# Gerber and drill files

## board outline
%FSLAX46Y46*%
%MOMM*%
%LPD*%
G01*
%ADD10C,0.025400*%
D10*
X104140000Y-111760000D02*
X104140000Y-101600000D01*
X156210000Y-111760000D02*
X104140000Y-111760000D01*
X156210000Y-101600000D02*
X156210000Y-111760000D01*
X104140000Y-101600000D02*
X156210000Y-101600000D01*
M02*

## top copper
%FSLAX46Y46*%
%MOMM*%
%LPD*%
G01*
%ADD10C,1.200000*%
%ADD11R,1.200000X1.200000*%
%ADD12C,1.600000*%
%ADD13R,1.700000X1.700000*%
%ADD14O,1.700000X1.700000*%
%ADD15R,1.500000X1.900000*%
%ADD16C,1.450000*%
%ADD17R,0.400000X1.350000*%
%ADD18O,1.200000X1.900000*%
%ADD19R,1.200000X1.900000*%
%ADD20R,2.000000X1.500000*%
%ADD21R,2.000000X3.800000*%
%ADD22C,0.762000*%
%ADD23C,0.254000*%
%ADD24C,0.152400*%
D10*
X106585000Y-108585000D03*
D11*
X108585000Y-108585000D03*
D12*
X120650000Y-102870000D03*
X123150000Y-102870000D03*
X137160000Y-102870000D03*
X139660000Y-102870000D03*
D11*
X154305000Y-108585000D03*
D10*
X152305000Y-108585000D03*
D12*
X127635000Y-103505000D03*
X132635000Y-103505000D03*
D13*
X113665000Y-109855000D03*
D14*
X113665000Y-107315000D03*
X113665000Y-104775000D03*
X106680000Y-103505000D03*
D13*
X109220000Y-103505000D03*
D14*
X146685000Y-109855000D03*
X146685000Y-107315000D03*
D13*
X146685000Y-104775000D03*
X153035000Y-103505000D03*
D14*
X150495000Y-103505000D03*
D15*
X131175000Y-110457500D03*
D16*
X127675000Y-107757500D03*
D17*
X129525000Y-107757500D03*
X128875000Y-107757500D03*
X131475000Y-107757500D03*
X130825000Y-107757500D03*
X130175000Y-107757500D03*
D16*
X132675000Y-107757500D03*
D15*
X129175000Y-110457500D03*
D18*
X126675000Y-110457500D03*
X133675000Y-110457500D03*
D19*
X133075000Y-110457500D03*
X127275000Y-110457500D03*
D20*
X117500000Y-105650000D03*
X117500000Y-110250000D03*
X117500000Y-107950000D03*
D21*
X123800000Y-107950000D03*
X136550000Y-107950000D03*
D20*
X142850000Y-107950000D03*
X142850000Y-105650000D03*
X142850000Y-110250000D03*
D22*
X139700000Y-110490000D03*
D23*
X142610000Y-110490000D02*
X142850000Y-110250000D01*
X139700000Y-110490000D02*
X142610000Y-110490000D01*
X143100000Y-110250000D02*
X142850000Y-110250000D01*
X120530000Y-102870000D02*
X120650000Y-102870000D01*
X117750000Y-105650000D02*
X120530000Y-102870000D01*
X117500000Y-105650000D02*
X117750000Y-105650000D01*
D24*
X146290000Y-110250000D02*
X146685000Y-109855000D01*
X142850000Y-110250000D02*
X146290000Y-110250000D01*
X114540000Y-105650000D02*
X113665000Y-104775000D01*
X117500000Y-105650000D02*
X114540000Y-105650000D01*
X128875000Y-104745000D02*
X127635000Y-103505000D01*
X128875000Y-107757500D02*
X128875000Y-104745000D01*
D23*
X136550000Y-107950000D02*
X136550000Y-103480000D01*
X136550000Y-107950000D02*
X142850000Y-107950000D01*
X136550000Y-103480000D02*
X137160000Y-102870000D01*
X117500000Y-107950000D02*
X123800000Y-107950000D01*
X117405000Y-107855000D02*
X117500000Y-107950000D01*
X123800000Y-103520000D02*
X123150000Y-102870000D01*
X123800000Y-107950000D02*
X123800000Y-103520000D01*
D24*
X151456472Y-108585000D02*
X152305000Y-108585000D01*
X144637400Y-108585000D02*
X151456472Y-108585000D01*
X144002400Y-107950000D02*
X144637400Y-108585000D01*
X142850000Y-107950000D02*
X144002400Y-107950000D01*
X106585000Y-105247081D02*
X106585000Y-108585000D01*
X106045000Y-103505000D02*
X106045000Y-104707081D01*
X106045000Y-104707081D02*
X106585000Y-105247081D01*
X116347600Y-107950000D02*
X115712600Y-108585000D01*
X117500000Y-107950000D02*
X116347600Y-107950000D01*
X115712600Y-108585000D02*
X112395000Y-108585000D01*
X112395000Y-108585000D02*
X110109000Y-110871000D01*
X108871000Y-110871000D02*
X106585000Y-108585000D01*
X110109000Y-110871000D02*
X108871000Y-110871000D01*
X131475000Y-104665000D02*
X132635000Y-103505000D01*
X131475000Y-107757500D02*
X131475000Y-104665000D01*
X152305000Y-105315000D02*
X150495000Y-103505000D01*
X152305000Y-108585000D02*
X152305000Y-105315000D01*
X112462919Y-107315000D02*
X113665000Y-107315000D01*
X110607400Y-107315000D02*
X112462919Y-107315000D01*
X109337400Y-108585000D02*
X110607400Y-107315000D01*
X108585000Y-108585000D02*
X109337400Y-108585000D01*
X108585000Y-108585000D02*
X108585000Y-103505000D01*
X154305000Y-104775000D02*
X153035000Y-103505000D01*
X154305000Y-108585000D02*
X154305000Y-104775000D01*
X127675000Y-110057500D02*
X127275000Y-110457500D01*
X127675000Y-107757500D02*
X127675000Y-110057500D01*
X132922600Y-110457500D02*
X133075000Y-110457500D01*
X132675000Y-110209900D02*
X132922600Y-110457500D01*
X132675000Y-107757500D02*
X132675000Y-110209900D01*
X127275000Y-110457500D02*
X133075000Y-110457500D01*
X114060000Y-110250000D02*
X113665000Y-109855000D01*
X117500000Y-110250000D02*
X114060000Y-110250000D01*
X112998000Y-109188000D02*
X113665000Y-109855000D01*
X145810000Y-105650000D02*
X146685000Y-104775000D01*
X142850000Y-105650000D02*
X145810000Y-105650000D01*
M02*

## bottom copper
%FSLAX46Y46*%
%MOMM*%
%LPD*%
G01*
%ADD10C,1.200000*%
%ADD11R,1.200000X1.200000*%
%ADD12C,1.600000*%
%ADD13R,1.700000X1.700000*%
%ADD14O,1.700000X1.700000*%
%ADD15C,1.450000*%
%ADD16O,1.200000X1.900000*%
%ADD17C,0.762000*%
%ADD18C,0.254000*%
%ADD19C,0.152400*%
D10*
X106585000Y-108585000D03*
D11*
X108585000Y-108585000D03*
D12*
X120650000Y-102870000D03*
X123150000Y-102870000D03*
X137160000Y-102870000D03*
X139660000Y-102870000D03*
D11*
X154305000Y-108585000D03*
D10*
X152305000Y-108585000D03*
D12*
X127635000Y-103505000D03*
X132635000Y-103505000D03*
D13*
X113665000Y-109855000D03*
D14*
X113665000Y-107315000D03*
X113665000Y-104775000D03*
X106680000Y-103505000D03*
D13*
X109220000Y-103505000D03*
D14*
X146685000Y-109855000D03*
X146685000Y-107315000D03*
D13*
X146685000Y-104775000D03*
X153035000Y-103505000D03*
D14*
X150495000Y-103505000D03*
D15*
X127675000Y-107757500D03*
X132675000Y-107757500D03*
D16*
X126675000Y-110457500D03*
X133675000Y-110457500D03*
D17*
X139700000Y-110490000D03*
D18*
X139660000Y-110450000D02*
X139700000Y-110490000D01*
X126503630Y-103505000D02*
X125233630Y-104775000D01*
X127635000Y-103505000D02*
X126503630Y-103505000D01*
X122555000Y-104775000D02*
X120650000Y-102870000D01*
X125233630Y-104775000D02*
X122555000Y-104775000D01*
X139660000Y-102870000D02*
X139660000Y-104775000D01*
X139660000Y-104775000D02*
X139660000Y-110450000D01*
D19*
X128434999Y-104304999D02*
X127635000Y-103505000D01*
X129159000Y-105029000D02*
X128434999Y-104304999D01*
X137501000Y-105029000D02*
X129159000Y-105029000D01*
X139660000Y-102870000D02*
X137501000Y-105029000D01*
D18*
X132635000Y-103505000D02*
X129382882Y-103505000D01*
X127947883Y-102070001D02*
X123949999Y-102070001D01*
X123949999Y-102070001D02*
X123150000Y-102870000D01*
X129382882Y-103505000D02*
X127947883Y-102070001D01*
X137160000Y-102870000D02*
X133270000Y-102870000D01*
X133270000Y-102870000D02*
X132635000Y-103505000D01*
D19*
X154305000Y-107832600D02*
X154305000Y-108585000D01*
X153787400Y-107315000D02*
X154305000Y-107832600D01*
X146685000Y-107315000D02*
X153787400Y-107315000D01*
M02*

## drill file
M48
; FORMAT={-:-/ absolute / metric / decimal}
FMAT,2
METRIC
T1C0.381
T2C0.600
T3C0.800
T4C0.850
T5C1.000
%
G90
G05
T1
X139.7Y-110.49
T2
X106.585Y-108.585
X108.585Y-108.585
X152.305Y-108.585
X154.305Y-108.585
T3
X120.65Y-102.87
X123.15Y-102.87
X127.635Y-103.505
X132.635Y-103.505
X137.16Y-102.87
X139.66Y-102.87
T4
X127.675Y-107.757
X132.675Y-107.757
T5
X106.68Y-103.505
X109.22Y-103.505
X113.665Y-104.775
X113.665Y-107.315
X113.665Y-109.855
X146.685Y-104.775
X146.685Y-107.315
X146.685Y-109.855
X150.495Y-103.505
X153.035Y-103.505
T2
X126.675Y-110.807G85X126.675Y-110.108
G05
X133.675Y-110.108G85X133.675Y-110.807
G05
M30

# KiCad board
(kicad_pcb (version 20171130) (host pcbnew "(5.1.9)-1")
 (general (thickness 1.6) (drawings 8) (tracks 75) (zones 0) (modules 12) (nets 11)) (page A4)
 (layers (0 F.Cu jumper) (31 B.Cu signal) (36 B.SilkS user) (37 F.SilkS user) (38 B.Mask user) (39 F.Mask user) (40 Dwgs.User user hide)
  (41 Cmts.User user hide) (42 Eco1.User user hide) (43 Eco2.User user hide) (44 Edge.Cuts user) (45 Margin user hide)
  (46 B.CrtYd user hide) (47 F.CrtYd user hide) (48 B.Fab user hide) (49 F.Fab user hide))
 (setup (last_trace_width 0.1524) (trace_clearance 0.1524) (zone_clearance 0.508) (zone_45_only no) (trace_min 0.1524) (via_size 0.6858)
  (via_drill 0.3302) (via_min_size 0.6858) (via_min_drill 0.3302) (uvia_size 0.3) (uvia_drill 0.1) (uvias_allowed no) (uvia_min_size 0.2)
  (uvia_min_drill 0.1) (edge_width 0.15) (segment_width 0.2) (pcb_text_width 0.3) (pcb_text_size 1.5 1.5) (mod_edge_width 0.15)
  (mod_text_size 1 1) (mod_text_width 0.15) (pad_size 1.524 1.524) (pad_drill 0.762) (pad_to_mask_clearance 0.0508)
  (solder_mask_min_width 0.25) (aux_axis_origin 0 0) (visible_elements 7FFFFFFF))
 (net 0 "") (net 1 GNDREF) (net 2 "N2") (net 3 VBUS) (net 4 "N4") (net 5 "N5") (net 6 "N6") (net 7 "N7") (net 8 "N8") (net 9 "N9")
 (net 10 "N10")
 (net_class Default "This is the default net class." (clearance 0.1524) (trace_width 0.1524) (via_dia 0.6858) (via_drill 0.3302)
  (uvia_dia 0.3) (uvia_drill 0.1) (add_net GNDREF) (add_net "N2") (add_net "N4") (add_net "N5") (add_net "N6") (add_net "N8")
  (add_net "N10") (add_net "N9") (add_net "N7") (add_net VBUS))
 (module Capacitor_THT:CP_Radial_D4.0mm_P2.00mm (layer F.Cu) (at 108.585 108.585 180)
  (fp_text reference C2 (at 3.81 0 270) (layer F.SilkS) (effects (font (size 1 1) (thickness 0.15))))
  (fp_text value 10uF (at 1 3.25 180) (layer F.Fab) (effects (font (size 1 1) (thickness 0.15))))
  (pad 2 thru_hole circle (at 2 0 180) (size 1.2 1.2) (drill 0.6) (layers *.Cu *.Mask) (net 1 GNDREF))
  (pad 1 thru_hole rect (at 0 0 180) (size 1.2 1.2) (drill 0.6) (layers *.Cu *.Mask) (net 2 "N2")))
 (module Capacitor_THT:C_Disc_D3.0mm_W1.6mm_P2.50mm (layer F.Cu) (at 120.65 102.87)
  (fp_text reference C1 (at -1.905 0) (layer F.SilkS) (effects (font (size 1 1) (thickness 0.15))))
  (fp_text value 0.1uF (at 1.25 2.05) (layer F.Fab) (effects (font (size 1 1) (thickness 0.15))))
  (pad 1 thru_hole circle (at 0 0) (size 1.6 1.6) (drill 0.8) (layers *.Cu *.Mask) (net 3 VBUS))
  (pad 2 thru_hole circle (at 2.5 0) (size 1.6 1.6) (drill 0.8) (layers *.Cu *.Mask) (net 1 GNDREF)))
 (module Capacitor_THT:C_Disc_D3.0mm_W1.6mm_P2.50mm (layer F.Cu) (at 139.66 102.87 180)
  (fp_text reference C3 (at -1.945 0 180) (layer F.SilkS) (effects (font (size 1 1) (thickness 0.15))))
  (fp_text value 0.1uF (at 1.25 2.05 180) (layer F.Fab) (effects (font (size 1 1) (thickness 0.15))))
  (pad 2 thru_hole circle (at 2.5 0 180) (size 1.6 1.6) (drill 0.8) (layers *.Cu *.Mask) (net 1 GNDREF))
  (pad 1 thru_hole circle (at 0 0 180) (size 1.6 1.6) (drill 0.8) (layers *.Cu *.Mask) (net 3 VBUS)))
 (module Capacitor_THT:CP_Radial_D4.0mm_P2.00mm (layer F.Cu) (at 154.305 108.585 180)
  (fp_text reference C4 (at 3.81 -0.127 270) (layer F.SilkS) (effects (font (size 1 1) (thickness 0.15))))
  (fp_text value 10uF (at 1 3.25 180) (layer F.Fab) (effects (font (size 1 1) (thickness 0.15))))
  (pad 1 thru_hole rect (at 0 0 180) (size 1.2 1.2) (drill 0.6) (layers *.Cu *.Mask) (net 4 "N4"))
  (pad 2 thru_hole circle (at 2 0 180) (size 1.2 1.2) (drill 0.6) (layers *.Cu *.Mask) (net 1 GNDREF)))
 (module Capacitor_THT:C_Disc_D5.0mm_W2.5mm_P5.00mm (layer F.Cu) (at 127.635 103.505)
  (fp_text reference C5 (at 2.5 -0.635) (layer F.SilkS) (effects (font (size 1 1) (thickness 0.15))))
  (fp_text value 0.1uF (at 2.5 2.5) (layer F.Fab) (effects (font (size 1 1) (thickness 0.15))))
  (pad 1 thru_hole circle (at 0 0) (size 1.6 1.6) (drill 0.8) (layers *.Cu *.Mask) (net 3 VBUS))
  (pad 2 thru_hole circle (at 5 0) (size 1.6 1.6) (drill 0.8) (layers *.Cu *.Mask) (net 1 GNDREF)))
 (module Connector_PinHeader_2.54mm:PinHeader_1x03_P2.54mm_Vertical (layer F.Cu) (at 113.665 109.855 180)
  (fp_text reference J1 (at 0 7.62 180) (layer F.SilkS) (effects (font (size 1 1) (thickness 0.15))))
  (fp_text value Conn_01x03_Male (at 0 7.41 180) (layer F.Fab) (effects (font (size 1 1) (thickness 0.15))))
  (pad 1 thru_hole rect (at 0 0 180) (size 1.7 1.7) (drill 1) (layers *.Cu *.Mask) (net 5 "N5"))
  (pad 2 thru_hole oval (at 0 2.54 180) (size 1.7 1.7) (drill 1) (layers *.Cu *.Mask) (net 2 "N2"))
  (pad 3 thru_hole oval (at 0 5.08 180) (size 1.7 1.7) (drill 1) (layers *.Cu *.Mask) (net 3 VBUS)))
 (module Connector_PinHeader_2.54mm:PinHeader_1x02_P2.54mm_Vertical (layer B.Cu) (at 109.22 103.505 90)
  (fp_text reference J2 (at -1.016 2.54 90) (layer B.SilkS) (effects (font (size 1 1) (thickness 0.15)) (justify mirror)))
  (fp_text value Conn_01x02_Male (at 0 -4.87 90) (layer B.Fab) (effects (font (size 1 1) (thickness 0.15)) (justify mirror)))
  (pad 2 thru_hole oval (at 0 -2.54 90) (size 1.7 1.7) (drill 1) (layers *.Cu *.Mask) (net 1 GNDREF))
  (pad 1 thru_hole rect (at 0 0 90) (size 1.7 1.7) (drill 1) (layers *.Cu *.Mask) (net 2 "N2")))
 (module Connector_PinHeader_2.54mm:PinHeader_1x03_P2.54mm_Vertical (layer F.Cu) (at 146.685 104.775)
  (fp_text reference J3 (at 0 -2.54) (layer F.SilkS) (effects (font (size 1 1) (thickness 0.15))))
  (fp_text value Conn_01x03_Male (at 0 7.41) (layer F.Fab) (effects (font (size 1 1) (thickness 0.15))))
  (pad 3 thru_hole oval (at 0 5.08) (size 1.7 1.7) (drill 1) (layers *.Cu *.Mask) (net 3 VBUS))
  (pad 2 thru_hole oval (at 0 2.54) (size 1.7 1.7) (drill 1) (layers *.Cu *.Mask) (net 4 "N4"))
  (pad 1 thru_hole rect (at 0 0) (size 1.7 1.7) (drill 1) (layers *.Cu *.Mask) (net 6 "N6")))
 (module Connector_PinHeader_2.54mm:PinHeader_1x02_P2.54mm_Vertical (layer B.Cu) (at 153.035 103.505 90)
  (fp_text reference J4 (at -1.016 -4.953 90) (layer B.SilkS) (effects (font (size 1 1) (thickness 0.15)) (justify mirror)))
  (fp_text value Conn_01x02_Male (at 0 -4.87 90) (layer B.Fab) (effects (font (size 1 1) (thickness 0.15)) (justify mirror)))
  (pad 1 thru_hole rect (at 0 0 90) (size 1.7 1.7) (drill 1) (layers *.Cu *.Mask) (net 4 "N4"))
  (pad 2 thru_hole oval (at 0 -2.54 90) (size 1.7 1.7) (drill 1) (layers *.Cu *.Mask) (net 1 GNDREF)))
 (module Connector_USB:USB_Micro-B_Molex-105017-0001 (layer F.Cu) (at 130.175 109.22)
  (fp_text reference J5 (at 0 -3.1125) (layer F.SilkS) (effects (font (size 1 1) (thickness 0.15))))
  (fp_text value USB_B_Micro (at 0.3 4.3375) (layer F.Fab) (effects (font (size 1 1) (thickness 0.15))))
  (pad 6 smd rect (at 1 1.2375) (size 1.5 1.9) (layers F.Cu F.Paste F.Mask) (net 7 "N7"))
  (pad 6 thru_hole circle (at -2.5 -1.4625) (size 1.45 1.45) (drill 0.85) (layers *.Cu *.Mask) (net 7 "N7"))
  (pad 2 smd rect (at -0.65 -1.4625) (size 0.4 1.35) (layers F.Cu F.Paste F.Mask) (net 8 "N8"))
  (pad 1 smd rect (at -1.3 -1.4625) (size 0.4 1.35) (layers F.Cu F.Paste F.Mask) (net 3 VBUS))
  (pad 5 smd rect (at 1.3 -1.4625) (size 0.4 1.35) (layers F.Cu F.Paste F.Mask) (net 1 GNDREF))
  (pad 4 smd rect (at 0.65 -1.4625) (size 0.4 1.35) (layers F.Cu F.Paste F.Mask) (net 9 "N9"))
  (pad 3 smd rect (at 0 -1.4625) (size 0.4 1.35) (layers F.Cu F.Paste F.Mask) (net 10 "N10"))
  (pad 6 thru_hole circle (at 2.5 -1.4625) (size 1.45 1.45) (drill 0.85) (layers *.Cu *.Mask) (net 7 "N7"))
  (pad 6 smd rect (at -1 1.2375) (size 1.5 1.9) (layers F.Cu F.Paste F.Mask) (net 7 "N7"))
  (pad 6 thru_hole oval (at -3.5 1.2375 180) (size 1.2 1.9) (drill oval 0.6 1.3) (layers *.Cu *.Mask) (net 7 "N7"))
  (pad 6 thru_hole oval (at 3.5 1.2375) (size 1.2 1.9) (drill oval 0.6 1.3) (layers *.Cu *.Mask) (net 7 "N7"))
  (pad 6 smd rect (at 2.9 1.2375) (size 1.2 1.9) (layers F.Cu F.Mask) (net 7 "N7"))
  (pad 6 smd rect (at -2.9 1.2375) (size 1.2 1.9) (layers F.Cu F.Mask) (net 7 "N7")))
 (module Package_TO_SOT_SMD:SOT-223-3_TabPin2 (layer F.Cu) (at 120.65 107.95)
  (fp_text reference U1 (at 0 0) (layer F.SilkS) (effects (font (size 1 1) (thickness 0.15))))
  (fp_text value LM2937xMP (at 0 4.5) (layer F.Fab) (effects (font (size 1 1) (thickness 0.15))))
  (pad 1 smd rect (at -3.15 -2.3) (size 2 1.5) (layers F.Cu F.Paste F.Mask) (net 3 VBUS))
  (pad 3 smd rect (at -3.15 2.3) (size 2 1.5) (layers F.Cu F.Paste F.Mask) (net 5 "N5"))
  (pad 2 smd rect (at -3.15 0) (size 2 1.5) (layers F.Cu F.Paste F.Mask) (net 1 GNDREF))
  (pad 2 smd rect (at 3.15 0) (size 2 3.8) (layers F.Cu F.Paste F.Mask) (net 1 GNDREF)))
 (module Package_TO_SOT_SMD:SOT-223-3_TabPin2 (layer F.Cu) (at 139.7 107.95 180)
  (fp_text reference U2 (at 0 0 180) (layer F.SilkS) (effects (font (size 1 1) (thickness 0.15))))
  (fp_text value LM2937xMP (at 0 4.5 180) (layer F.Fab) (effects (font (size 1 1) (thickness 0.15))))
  (pad 2 smd rect (at 3.15 0 180) (size 2 3.8) (layers F.Cu F.Paste F.Mask) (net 1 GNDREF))
  (pad 2 smd rect (at -3.15 0 180) (size 2 1.5) (layers F.Cu F.Paste F.Mask) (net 1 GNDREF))
  (pad 3 smd rect (at -3.15 2.3 180) (size 2 1.5) (layers F.Cu F.Paste F.Mask) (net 6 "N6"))
  (pad 1 smd rect (at -3.15 -2.3 180) (size 2 1.5) (layers F.Cu F.Paste F.Mask) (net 3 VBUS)))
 (gr_line (start 104.14 111.76) (end 104.14 101.6) (layer Edge.Cuts) (width 0.0254))
 (gr_line (start 156.21 111.76) (end 104.14 111.76) (layer Edge.Cuts) (width 0.0254))
 (gr_line (start 156.21 101.6) (end 156.21 111.76) (layer Edge.Cuts) (width 0.0254))
 (gr_line (start 104.14 101.6) (end 156.21 101.6) (layer Edge.Cuts) (width 0.0254))
 (via (at 139.7 110.49) (size 0.762) (drill 0.381) (layers F.Cu B.Cu) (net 3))
 (segment (start 139.66 110.45) (end 139.7 110.49) (width 0.254) (layer B.Cu) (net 3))
 (segment (start 142.61 110.49) (end 142.85 110.25) (width 0.254) (layer F.Cu) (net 3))
 (segment (start 139.7 110.49) (end 142.61 110.49) (width 0.254) (layer F.Cu) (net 3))
 (segment (start 143.1 110.25) (end 142.85 110.25) (width 0.254) (layer F.Cu) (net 3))
 (segment (start 126.50363 103.505) (end 125.23363 104.775) (width 0.254) (layer B.Cu) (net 3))
 (segment (start 127.635 103.505) (end 126.50363 103.505) (width 0.254) (layer B.Cu) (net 3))
 (segment (start 122.555 104.775) (end 120.65 102.87) (width 0.254) (layer B.Cu) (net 3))
 (segment (start 125.23363 104.775) (end 122.555 104.775) (width 0.254) (layer B.Cu) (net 3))
 (segment (start 120.53 102.87) (end 120.65 102.87) (width 0.254) (layer F.Cu) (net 3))
 (segment (start 117.75 105.65) (end 120.53 102.87) (width 0.254) (layer F.Cu) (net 3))
 (segment (start 117.5 105.65) (end 117.75 105.65) (width 0.254) (layer F.Cu) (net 3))
 (segment (start 139.66 102.87) (end 139.66 104.775) (width 0.254) (layer B.Cu) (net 3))
 (segment (start 139.66 104.775) (end 139.66 110.45) (width 0.254) (layer B.Cu) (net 3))
 (segment (start 128.434999 104.304999) (end 127.635 103.505) (width 0.1524) (layer B.Cu) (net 3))
 (segment (start 129.159 105.029) (end 128.434999 104.304999) (width 0.1524) (layer B.Cu) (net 3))
 (segment (start 137.501 105.029) (end 129.159 105.029) (width 0.1524) (layer B.Cu) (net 3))
 (segment (start 139.66 102.87) (end 137.501 105.029) (width 0.1524) (layer B.Cu) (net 3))
 (segment (start 146.29 110.25) (end 146.685 109.855) (width 0.1524) (layer F.Cu) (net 3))
 (segment (start 142.85 110.25) (end 146.29 110.25) (width 0.1524) (layer F.Cu) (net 3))
 (segment (start 114.54 105.65) (end 113.665 104.775) (width 0.1524) (layer F.Cu) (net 3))
 (segment (start 117.5 105.65) (end 114.54 105.65) (width 0.1524) (layer F.Cu) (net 3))
 (segment (start 128.875 104.745) (end 127.635 103.505) (width 0.1524) (layer F.Cu) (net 3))
 (segment (start 128.875 107.7575) (end 128.875 104.745) (width 0.1524) (layer F.Cu) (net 3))
 (segment (start 136.55 107.95) (end 136.55 103.48) (width 0.254) (layer F.Cu) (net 1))
 (segment (start 136.55 107.95) (end 142.85 107.95) (width 0.254) (layer F.Cu) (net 1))
 (segment (start 132.635 103.505) (end 129.382882 103.505) (width 0.254) (layer B.Cu) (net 1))
 (segment (start 127.947883 102.070001) (end 123.949999 102.070001) (width 0.254) (layer B.Cu) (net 1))
 (segment (start 123.949999 102.070001) (end 123.15 102.87) (width 0.254) (layer B.Cu) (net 1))
 (segment (start 129.382882 103.505) (end 127.947883 102.070001) (width 0.254) (layer B.Cu) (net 1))
 (segment (start 136.55 103.48) (end 137.16 102.87) (width 0.254) (layer F.Cu) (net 1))
 (segment (start 137.16 102.87) (end 133.27 102.87) (width 0.254) (layer B.Cu) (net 1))
 (segment (start 117.5 107.95) (end 123.8 107.95) (width 0.254) (layer F.Cu) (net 1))
 (segment (start 133.27 102.87) (end 132.635 103.505) (width 0.254) (layer B.Cu) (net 1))
 (segment (start 117.405 107.855) (end 117.5 107.95) (width 0.254) (layer F.Cu) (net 1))
 (segment (start 123.8 103.52) (end 123.15 102.87) (width 0.254) (layer F.Cu) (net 1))
 (segment (start 123.8 107.95) (end 123.8 103.52) (width 0.254) (layer F.Cu) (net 1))
 (segment (start 151.456472 108.585) (end 152.305 108.585) (width 0.1524) (layer F.Cu) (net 1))
 (segment (start 144.6374 108.585) (end 151.456472 108.585) (width 0.1524) (layer F.Cu) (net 1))
 (segment (start 144.0024 107.95) (end 144.6374 108.585) (width 0.1524) (layer F.Cu) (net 1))
 (segment (start 142.85 107.95) (end 144.0024 107.95) (width 0.1524) (layer F.Cu) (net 1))
 (segment (start 106.585 105.247081) (end 106.585 108.585) (width 0.1524) (layer F.Cu) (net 1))
 (segment (start 106.045 103.505) (end 106.045 104.707081) (width 0.1524) (layer F.Cu) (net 1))
 (segment (start 106.045 104.707081) (end 106.585 105.247081) (width 0.1524) (layer F.Cu) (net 1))
 (segment (start 116.3476 107.95) (end 115.7126 108.585) (width 0.1524) (layer F.Cu) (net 1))
 (segment (start 117.5 107.95) (end 116.3476 107.95) (width 0.1524) (layer F.Cu) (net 1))
 (segment (start 115.7126 108.585) (end 112.395 108.585) (width 0.1524) (layer F.Cu) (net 1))
 (segment (start 112.395 108.585) (end 110.109 110.871) (width 0.1524) (layer F.Cu) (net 1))
 (segment (start 108.871 110.871) (end 106.585 108.585) (width 0.1524) (layer F.Cu) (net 1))
 (segment (start 110.109 110.871) (end 108.871 110.871) (width 0.1524) (layer F.Cu) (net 1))
 (segment (start 131.475 104.665) (end 132.635 103.505) (width 0.1524) (layer F.Cu) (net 1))
 (segment (start 131.475 107.7575) (end 131.475 104.665) (width 0.1524) (layer F.Cu) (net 1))
 (segment (start 152.305 105.315) (end 150.495 103.505) (width 0.1524) (layer F.Cu) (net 1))
 (segment (start 152.305 108.585) (end 152.305 105.315) (width 0.1524) (layer F.Cu) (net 1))
 (segment (start 112.462919 107.315) (end 113.665 107.315) (width 0.1524) (layer F.Cu) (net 2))
 (segment (start 110.6074 107.315) (end 112.462919 107.315) (width 0.1524) (layer F.Cu) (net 2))
 (segment (start 109.3374 108.585) (end 110.6074 107.315) (width 0.1524) (layer F.Cu) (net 2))
 (segment (start 108.585 108.585) (end 109.3374 108.585) (width 0.1524) (layer F.Cu) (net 2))
 (segment (start 108.585 108.585) (end 108.585 103.505) (width 0.1524) (layer F.Cu) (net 2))
 (segment (start 154.305 107.8326) (end 154.305 108.585) (width 0.1524) (layer B.Cu) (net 4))
 (segment (start 153.7874 107.315) (end 154.305 107.8326) (width 0.1524) (layer B.Cu) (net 4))
 (segment (start 146.685 107.315) (end 153.7874 107.315) (width 0.1524) (layer B.Cu) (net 4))
 (segment (start 154.305 104.775) (end 153.035 103.505) (width 0.1524) (layer F.Cu) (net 4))
 (segment (start 154.305 108.585) (end 154.305 104.775) (width 0.1524) (layer F.Cu) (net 4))
 (segment (start 127.675 110.0575) (end 127.275 110.4575) (width 0.1524) (layer F.Cu) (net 7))
 (segment (start 127.675 107.7575) (end 127.675 110.0575) (width 0.1524) (layer F.Cu) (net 7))
 (segment (start 132.9226 110.4575) (end 133.075 110.4575) (width 0.1524) (layer F.Cu) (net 7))
 (segment (start 132.675 110.2099) (end 132.9226 110.4575) (width 0.1524) (layer F.Cu) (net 7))
 (segment (start 132.675 107.7575) (end 132.675 110.2099) (width 0.1524) (layer F.Cu) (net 7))
 (segment (start 127.275 110.4575) (end 133.075 110.4575) (width 0.1524) (layer F.Cu) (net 7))
 (segment (start 114.06 110.25) (end 113.665 109.855) (width 0.1524) (layer F.Cu) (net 5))
 (segment (start 117.5 110.25) (end 114.06 110.25) (width 0.1524) (layer F.Cu) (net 5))
 (segment (start 112.998 109.188) (end 113.665 109.855) (width 0.1524) (layer F.Cu) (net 5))
 (segment (start 145.81 105.65) (end 146.685 104.775) (width 0.1524) (layer F.Cu) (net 6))
 (segment (start 142.85 105.65) (end 145.81 105.65) (width 0.1524) (layer F.Cu) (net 6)))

